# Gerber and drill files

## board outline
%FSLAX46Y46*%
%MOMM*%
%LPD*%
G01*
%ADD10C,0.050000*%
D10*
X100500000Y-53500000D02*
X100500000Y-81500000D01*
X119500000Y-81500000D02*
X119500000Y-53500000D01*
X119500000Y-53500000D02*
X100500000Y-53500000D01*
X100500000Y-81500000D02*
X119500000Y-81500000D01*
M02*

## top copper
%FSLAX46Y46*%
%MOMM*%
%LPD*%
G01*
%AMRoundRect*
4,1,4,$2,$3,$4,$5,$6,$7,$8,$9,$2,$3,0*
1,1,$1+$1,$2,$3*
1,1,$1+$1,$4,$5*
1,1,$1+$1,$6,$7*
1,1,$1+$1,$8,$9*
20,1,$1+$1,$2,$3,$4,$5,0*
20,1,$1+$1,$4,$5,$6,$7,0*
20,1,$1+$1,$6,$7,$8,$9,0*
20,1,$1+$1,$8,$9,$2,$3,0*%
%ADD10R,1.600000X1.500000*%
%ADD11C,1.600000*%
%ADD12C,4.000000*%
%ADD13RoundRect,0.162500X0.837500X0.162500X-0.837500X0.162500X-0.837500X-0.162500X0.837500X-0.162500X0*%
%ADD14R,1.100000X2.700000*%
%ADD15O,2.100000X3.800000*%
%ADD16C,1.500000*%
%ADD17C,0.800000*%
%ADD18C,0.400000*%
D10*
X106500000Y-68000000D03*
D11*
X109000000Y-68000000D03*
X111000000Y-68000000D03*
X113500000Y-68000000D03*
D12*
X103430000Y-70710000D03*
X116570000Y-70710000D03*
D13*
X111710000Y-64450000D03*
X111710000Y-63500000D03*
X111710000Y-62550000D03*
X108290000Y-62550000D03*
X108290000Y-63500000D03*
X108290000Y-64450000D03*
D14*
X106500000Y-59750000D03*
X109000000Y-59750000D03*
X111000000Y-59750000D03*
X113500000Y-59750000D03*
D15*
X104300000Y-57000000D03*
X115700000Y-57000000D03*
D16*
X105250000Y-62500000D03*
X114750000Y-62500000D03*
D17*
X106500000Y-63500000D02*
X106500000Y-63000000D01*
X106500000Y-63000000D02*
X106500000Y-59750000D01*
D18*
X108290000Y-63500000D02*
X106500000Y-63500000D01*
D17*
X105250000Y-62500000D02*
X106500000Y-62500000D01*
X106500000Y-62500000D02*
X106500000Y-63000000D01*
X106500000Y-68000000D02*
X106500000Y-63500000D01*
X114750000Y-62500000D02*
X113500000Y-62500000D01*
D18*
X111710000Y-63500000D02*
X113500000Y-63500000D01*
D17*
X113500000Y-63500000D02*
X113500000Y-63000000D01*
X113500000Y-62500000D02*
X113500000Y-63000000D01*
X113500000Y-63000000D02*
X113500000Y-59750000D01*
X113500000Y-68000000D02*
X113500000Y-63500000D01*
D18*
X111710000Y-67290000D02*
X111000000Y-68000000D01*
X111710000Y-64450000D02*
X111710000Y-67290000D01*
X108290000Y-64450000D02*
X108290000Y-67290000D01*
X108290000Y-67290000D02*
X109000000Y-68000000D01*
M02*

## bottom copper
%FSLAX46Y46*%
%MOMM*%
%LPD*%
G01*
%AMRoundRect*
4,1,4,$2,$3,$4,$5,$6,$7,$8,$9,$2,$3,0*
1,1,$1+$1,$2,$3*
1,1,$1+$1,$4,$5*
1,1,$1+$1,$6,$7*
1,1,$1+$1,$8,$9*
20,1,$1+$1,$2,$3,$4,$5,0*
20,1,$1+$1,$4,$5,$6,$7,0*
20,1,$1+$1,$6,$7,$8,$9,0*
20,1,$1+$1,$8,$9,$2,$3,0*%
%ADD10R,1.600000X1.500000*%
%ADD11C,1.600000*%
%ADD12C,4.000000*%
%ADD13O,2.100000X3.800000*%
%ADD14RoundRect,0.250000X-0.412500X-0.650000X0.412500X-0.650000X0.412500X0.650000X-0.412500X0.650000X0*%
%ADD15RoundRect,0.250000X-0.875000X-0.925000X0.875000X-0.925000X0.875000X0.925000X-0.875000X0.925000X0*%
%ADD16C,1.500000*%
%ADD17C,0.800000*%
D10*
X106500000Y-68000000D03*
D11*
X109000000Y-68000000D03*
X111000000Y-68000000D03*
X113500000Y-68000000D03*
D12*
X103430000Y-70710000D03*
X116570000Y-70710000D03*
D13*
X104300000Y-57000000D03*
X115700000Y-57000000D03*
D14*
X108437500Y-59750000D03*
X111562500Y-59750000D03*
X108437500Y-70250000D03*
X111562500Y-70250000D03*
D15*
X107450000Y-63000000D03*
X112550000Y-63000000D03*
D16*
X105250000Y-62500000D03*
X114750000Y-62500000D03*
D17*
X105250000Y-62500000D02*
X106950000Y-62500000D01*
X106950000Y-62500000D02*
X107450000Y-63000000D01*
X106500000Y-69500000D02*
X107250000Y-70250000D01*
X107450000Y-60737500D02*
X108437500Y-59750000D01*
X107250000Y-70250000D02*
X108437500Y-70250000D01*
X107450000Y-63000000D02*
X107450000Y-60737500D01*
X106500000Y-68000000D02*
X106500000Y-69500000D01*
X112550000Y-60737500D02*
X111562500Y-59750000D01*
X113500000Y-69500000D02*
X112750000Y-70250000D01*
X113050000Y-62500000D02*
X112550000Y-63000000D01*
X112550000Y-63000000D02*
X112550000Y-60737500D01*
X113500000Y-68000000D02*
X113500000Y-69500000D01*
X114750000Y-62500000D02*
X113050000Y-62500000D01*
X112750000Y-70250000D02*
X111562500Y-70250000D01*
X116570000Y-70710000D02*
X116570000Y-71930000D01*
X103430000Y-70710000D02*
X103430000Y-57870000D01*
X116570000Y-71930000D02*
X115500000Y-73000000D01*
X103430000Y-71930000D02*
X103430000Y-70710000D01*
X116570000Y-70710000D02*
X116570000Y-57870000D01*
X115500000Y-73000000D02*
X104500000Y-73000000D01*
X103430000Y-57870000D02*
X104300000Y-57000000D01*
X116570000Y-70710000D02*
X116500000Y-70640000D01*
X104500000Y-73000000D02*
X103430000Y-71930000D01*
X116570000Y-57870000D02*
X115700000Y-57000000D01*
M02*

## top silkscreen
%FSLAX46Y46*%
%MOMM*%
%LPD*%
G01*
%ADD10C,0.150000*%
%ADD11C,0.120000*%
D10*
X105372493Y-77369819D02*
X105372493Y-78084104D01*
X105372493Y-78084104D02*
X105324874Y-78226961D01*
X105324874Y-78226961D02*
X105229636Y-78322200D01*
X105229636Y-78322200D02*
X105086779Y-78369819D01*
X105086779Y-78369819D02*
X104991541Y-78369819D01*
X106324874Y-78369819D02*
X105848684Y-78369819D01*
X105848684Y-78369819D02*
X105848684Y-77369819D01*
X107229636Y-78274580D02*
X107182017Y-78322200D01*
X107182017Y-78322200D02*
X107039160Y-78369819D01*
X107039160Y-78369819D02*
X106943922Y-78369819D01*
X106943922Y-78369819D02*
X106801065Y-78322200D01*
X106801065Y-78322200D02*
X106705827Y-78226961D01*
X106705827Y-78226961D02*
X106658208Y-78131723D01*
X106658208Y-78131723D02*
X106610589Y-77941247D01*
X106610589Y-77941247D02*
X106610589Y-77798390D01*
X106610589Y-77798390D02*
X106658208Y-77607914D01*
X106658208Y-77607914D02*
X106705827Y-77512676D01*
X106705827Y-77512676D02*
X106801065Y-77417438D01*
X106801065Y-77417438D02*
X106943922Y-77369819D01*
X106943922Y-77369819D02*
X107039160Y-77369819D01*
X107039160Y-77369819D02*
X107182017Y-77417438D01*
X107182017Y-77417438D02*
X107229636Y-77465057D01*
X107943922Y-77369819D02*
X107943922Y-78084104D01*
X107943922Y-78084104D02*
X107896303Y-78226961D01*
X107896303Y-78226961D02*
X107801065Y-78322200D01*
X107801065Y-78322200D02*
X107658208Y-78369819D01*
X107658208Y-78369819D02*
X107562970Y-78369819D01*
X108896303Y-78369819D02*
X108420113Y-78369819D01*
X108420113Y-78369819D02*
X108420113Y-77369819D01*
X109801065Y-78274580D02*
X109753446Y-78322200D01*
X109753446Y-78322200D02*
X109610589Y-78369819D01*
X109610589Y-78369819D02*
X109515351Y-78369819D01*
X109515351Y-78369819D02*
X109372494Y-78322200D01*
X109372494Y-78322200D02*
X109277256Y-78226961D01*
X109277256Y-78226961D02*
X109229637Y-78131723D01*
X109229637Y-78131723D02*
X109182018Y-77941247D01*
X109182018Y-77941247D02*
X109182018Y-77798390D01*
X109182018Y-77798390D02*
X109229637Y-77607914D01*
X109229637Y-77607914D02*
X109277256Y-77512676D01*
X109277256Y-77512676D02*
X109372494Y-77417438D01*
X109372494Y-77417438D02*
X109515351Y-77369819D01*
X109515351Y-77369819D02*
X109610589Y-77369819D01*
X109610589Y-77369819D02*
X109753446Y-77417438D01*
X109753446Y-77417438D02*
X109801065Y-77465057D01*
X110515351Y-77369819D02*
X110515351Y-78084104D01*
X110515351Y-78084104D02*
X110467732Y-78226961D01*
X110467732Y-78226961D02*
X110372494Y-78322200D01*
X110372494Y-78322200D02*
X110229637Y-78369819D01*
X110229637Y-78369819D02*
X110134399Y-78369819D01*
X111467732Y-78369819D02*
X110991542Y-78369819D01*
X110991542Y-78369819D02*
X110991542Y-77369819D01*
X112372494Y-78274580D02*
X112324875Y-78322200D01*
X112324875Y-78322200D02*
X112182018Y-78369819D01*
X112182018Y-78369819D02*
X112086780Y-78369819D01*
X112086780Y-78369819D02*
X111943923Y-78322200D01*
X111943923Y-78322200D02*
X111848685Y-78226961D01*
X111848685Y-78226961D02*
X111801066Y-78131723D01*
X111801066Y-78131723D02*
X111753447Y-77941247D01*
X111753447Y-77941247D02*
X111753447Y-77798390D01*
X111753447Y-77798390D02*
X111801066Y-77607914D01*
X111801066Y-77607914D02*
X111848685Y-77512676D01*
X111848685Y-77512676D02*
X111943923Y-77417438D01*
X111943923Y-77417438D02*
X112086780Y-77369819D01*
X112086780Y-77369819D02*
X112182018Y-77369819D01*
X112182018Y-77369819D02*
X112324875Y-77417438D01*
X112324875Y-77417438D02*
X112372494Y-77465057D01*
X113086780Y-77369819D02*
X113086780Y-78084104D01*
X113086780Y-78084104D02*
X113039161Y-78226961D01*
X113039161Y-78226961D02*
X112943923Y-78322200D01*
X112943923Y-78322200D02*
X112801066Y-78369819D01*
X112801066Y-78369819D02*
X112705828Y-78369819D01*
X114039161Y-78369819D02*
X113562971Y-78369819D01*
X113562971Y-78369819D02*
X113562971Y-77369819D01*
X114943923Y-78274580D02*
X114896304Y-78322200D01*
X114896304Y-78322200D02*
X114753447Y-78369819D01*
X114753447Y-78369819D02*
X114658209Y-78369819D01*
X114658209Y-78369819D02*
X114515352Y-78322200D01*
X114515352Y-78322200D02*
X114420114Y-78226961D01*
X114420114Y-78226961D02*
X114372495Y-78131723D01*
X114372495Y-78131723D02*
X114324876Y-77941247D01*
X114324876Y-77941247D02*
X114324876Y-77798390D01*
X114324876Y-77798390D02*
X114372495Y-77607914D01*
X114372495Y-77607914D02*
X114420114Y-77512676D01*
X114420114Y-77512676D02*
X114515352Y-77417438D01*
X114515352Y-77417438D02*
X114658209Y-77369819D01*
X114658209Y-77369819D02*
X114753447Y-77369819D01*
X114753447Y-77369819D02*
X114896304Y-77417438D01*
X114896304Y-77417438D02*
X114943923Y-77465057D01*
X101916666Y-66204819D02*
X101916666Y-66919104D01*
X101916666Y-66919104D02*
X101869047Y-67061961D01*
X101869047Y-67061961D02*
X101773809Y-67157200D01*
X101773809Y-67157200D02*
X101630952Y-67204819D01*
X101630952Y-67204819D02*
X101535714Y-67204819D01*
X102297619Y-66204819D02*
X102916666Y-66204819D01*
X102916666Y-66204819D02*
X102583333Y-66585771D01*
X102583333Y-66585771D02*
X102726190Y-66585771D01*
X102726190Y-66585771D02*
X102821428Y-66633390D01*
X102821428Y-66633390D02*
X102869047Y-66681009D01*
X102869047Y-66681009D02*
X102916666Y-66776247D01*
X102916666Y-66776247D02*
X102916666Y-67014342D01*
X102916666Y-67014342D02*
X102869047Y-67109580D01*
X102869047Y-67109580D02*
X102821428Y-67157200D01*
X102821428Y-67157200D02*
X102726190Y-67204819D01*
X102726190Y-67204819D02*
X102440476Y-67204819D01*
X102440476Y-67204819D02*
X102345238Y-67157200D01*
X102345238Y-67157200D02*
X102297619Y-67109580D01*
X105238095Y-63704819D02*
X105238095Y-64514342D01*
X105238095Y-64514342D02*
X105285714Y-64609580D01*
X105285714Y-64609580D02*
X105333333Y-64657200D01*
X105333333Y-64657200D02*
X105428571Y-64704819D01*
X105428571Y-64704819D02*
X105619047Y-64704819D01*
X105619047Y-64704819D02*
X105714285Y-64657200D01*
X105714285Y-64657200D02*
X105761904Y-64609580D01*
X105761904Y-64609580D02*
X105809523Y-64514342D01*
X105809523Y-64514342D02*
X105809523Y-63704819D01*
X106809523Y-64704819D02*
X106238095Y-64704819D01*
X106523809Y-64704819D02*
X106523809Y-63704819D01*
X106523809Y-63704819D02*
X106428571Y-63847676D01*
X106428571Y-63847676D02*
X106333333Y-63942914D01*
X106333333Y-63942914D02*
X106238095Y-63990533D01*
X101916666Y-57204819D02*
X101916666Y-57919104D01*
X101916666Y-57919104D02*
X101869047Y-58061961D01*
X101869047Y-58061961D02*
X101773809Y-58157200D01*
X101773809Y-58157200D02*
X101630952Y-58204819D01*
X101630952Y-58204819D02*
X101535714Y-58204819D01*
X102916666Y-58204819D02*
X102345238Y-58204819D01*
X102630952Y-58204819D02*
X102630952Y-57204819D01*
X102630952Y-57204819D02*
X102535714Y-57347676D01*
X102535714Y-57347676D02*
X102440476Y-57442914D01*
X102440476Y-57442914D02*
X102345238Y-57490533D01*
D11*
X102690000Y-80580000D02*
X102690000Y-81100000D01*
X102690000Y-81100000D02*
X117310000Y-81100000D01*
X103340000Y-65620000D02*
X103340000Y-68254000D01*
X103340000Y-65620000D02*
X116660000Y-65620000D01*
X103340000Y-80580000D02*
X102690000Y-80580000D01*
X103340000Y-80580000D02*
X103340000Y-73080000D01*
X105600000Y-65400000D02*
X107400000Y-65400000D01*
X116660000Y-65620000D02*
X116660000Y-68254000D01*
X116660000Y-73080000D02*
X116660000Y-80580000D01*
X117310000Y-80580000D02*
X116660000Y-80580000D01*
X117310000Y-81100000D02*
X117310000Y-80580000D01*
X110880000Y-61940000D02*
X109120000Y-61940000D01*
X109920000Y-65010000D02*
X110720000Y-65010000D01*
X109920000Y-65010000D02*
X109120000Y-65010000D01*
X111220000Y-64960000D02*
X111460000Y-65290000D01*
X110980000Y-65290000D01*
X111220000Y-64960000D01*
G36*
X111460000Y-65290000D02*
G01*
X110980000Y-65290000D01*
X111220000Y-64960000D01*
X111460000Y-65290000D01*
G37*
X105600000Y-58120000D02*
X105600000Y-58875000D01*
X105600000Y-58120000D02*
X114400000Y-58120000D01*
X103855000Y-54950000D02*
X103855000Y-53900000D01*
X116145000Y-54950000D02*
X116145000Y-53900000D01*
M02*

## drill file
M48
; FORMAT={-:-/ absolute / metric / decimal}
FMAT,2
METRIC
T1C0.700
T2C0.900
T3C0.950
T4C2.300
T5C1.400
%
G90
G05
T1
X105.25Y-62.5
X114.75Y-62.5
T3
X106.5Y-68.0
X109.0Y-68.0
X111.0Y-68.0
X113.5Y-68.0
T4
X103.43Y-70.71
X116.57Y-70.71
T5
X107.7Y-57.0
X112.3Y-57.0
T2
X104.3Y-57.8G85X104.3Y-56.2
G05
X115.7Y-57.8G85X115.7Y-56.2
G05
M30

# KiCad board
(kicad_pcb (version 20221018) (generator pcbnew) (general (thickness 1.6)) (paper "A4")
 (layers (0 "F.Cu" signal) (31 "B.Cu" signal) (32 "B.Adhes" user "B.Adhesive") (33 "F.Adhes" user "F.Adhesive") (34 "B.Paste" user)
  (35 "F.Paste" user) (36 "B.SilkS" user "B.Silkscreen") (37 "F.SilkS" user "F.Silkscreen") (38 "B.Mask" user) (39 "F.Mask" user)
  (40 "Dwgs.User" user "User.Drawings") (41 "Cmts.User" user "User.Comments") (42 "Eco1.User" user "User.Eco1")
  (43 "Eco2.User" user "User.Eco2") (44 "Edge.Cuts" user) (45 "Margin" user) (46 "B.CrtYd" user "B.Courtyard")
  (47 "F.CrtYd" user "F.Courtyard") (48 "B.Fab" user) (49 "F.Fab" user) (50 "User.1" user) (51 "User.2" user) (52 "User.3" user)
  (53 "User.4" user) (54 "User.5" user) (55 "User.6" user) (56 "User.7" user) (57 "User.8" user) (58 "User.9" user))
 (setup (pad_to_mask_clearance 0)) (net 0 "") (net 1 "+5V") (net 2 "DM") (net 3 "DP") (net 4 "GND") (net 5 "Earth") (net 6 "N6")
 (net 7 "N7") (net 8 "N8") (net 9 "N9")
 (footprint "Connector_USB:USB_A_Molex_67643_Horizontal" (layer "F.Cu") (at 106.5 68)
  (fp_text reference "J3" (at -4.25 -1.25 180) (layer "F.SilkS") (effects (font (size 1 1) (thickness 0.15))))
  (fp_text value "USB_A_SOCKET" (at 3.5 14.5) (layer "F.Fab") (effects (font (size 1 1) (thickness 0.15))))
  (fp_line (start -3.81 12.58) (end -3.81 13.1) (stroke (width 0.12) (type solid)) (layer "F.SilkS"))
  (fp_line (start -3.81 13.1) (end 10.81 13.1) (stroke (width 0.12) (type solid)) (layer "F.SilkS"))
  (fp_line (start -3.16 -2.38) (end -3.16 0.254) (stroke (width 0.12) (type solid)) (layer "F.SilkS"))
  (fp_line (start -3.16 -2.38) (end 10.16 -2.38) (stroke (width 0.12) (type solid)) (layer "F.SilkS"))
  (fp_line (start -3.16 12.58) (end -3.81 12.58) (stroke (width 0.12) (type solid)) (layer "F.SilkS"))
  (fp_line (start -3.16 12.58) (end -3.16 5.08) (stroke (width 0.12) (type solid)) (layer "F.SilkS"))
  (fp_line (start -0.9 -2.6) (end 0.9 -2.6) (stroke (width 0.12) (type solid)) (layer "F.SilkS"))
  (fp_line (start 10.16 -2.38) (end 10.16 0.254) (stroke (width 0.12) (type solid)) (layer "F.SilkS"))
  (fp_line (start 10.16 5.08) (end 10.16 12.58) (stroke (width 0.12) (type solid)) (layer "F.SilkS"))
  (fp_line (start 10.81 12.58) (end 10.16 12.58) (stroke (width 0.12) (type solid)) (layer "F.SilkS"))
  (fp_line (start 10.81 13.1) (end 10.81 12.58) (stroke (width 0.12) (type solid)) (layer "F.SilkS"))
  (pad "1" thru_hole rect (at 0 0) (size 1.6 1.5) (drill 0.95) (layers "*.Cu" "*.Mask") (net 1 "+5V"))
  (pad "2" thru_hole circle (at 2.5 0) (size 1.6 1.6) (drill 0.95) (layers "*.Cu" "*.Mask") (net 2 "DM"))
  (pad "3" thru_hole circle (at 4.5 0) (size 1.6 1.6) (drill 0.95) (layers "*.Cu" "*.Mask") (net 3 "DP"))
  (pad "4" thru_hole circle (at 7 0) (size 1.6 1.6) (drill 0.95) (layers "*.Cu" "*.Mask") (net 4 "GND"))
  (pad "5" thru_hole circle (at -3.07 2.71) (size 4 4) (drill 2.3) (layers "*.Cu" "*.Mask") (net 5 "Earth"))
  (pad "5" thru_hole circle (at 10.07 2.71) (size 4 4) (drill 2.3) (layers "*.Cu" "*.Mask") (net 5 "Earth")))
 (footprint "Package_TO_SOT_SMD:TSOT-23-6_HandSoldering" (layer "F.Cu") (at 110 63.5 180)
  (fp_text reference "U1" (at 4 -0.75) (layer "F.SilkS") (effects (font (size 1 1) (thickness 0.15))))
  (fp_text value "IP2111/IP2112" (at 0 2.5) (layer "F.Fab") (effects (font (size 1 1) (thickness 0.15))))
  (fp_line (start -0.88 1.56) (end 0.88 1.56) (stroke (width 0.12) (type solid)) (layer "F.SilkS"))
  (fp_line (start 0.08 -1.51) (end -0.72 -1.51) (stroke (width 0.12) (type solid)) (layer "F.SilkS"))
  (fp_line (start 0.08 -1.51) (end 0.88 -1.51) (stroke (width 0.12) (type solid)) (layer "F.SilkS"))
  (fp_poly
   (pts (xy -1.22 -1.46) (xy -1.46 -1.79) (xy -0.98 -1.79) (xy -1.22 -1.46)) (stroke (width 0.12) (type solid)) (fill solid)
   (layer "F.SilkS"))
  (pad "1" smd roundrect (at -1.71 -0.95 180) (size 2 0.65) (layers "F.Cu" "F.Paste" "F.Mask") (roundrect_rratio 0.25) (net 3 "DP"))
  (pad "2" smd roundrect (at -1.71 0 180) (size 2 0.65) (layers "F.Cu" "F.Paste" "F.Mask") (roundrect_rratio 0.25) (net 4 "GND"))
  (pad "3" smd roundrect (at -1.71 0.95 180) (size 2 0.65) (layers "F.Cu" "F.Paste" "F.Mask") (roundrect_rratio 0.25) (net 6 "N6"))
  (pad "4" smd roundrect (at 1.71 0.95 180) (size 2 0.65) (layers "F.Cu" "F.Paste" "F.Mask") (roundrect_rratio 0.25) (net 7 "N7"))
  (pad "5" smd roundrect (at 1.71 0 180) (size 2 0.65) (layers "F.Cu" "F.Paste" "F.Mask") (roundrect_rratio 0.25) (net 1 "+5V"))
  (pad "6" smd roundrect (at 1.71 -0.95 180) (size 2 0.65) (layers "F.Cu" "F.Paste" "F.Mask") (roundrect_rratio 0.25) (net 2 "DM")))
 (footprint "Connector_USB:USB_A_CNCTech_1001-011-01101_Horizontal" (layer "F.Cu") (at 110 50.1 90)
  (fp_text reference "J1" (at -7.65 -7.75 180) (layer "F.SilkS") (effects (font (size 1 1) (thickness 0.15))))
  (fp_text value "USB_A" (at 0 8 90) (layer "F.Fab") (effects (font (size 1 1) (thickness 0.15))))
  (fp_line (start -8.02 -4.4) (end -8.775 -4.4) (stroke (width 0.12) (type solid)) (layer "F.SilkS"))
  (fp_line (start -8.02 -4.4) (end -8.02 4.4) (stroke (width 0.12) (type solid)) (layer "F.SilkS"))
  (fp_line (start -4.85 -6.145) (end -3.8 -6.145) (stroke (width 0.12) (type solid)) (layer "F.SilkS"))
  (fp_line (start -4.85 6.145) (end -3.8 6.145) (stroke (width 0.12) (type solid)) (layer "F.SilkS"))
  (pad "" np_thru_hole circle (at -6.9 -2.3 90) (size 1.1 1.1) (drill 1.4) (layers "F&B.Cu" "*.Mask"))
  (pad "" np_thru_hole circle (at -6.9 2.3 90) (size 1.1 1.1) (drill 1.4) (layers "F&B.Cu" "*.Mask"))
  (pad "1" smd rect (at -9.65 -3.5 90) (size 2.7 1.1) (layers "F.Cu" "F.Paste" "F.Mask") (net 1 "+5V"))
  (pad "2" smd rect (at -9.65 -1 90) (size 2.7 1.1) (layers "F.Cu" "F.Paste" "F.Mask") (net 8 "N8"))
  (pad "3" smd rect (at -9.65 1 90) (size 2.7 1.1) (layers "F.Cu" "F.Paste" "F.Mask") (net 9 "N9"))
  (pad "4" smd rect (at -9.65 3.5 90) (size 2.7 1.1) (layers "F.Cu" "F.Paste" "F.Mask") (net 4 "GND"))
  (pad "5" thru_hole oval (at -6.9 -5.7 90) (size 3.8 2.1) (drill oval 2.5 0.9) (layers "*.Cu" "*.Mask") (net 5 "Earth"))
  (pad "5" thru_hole oval (at -6.9 5.7 90) (size 3.8 2.1) (drill oval 2.5 0.9) (layers "*.Cu" "*.Mask") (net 5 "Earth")))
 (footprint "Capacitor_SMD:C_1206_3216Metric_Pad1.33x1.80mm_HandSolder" (layer "B.Cu") (at 110 59.75)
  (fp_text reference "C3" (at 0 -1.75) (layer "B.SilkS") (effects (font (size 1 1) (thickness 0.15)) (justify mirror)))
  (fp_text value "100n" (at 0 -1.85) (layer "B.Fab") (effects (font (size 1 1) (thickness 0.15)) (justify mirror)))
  (pad "1" smd roundrect (at -1.5625 0) (size 1.325 1.8) (layers "B.Cu" "B.Paste" "B.Mask") (roundrect_rratio 0.1886792453) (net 1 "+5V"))
  (pad "2" smd roundrect (at 1.5625 0) (size 1.325 1.8) (layers "B.Cu" "B.Paste" "B.Mask") (roundrect_rratio 0.1886792453) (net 4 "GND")))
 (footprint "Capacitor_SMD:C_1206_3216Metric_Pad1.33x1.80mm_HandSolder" (layer "B.Cu") (at 110 70.25)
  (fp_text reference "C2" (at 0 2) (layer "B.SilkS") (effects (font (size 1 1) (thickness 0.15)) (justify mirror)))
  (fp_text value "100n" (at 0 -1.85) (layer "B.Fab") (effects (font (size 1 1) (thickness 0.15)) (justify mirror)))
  (pad "1" smd roundrect (at -1.5625 0) (size 1.325 1.8) (layers "B.Cu" "B.Paste" "B.Mask") (roundrect_rratio 0.1886792453) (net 1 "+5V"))
  (pad "2" smd roundrect (at 1.5625 0) (size 1.325 1.8) (layers "B.Cu" "B.Paste" "B.Mask") (roundrect_rratio 0.1886792453) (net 4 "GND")))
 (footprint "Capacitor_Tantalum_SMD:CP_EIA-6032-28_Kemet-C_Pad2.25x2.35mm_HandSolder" (layer "B.Cu") (at 110 63)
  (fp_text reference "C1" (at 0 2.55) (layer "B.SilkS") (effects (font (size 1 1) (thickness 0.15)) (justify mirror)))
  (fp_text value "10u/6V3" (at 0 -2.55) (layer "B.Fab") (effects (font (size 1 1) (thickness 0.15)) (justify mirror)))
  (pad "1" smd roundrect (at -2.55 0) (size 2.25 2.35) (layers "B.Cu" "B.Paste" "B.Mask") (roundrect_rratio 0.1111111111) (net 1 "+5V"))
  (pad "2" smd roundrect (at 2.55 0) (size 2.25 2.35) (layers "B.Cu" "B.Paste" "B.Mask") (roundrect_rratio 0.1111111111) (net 4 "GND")))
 (gr_line (start 100.5 53.5) (end 100.5 81.5) (stroke (width 0.05) (type default)) (layer "Edge.Cuts"))
 (gr_line (start 119.5 81.5) (end 119.5 53.5) (stroke (width 0.05) (type default)) (layer "Edge.Cuts"))
 (gr_line (start 119.5 53.5) (end 100.5 53.5) (stroke (width 0.05) (type default)) (layer "Edge.Cuts"))
 (gr_line (start 100.5 81.5) (end 119.5 81.5) (stroke (width 0.05) (type default)) (layer "Edge.Cuts"))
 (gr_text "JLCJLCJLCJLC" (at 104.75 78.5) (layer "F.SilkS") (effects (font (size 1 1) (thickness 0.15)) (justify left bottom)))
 (segment (start 106.5 63.5) (end 106.5 63) (width 0.8) (layer "F.Cu") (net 1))
 (segment (start 106.5 63) (end 106.5 59.75) (width 0.8) (layer "F.Cu") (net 1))
 (segment (start 108.29 63.5) (end 106.5 63.5) (width 0.4) (layer "F.Cu") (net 1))
 (segment (start 105.25 62.5) (end 106.5 62.5) (width 0.8) (layer "F.Cu") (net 1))
 (segment (start 106.5 62.5) (end 106.5 63) (width 0.8) (layer "F.Cu") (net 1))
 (segment (start 106.5 68) (end 106.5 63.5) (width 0.8) (layer "F.Cu") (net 1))
 (via (at 105.25 62.5) (size 1.5) (drill 0.7) (layers "F.Cu" "B.Cu") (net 1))
 (segment (start 105.25 62.5) (end 106.95 62.5) (width 0.8) (layer "B.Cu") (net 1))
 (segment (start 106.95 62.5) (end 107.45 63) (width 0.8) (layer "B.Cu") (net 1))
 (segment (start 106.5 69.5) (end 107.25 70.25) (width 0.8) (layer "B.Cu") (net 1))
 (segment (start 107.45 60.7375) (end 108.4375 59.75) (width 0.8) (layer "B.Cu") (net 1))
 (segment (start 107.25 70.25) (end 108.4375 70.25) (width 0.8) (layer "B.Cu") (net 1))
 (segment (start 107.45 63) (end 107.45 60.7375) (width 0.8) (layer "B.Cu") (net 1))
 (segment (start 106.5 68) (end 106.5 69.5) (width 0.8) (layer "B.Cu") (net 1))
 (segment (start 114.75 62.5) (end 113.5 62.5) (width 0.8) (layer "F.Cu") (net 4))
 (segment (start 111.71 63.5) (end 113.5 63.5) (width 0.4) (layer "F.Cu") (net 4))
 (segment (start 113.5 63.5) (end 113.5 63) (width 0.8) (layer "F.Cu") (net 4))
 (segment (start 113.5 62.5) (end 113.5 63) (width 0.8) (layer "F.Cu") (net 4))
 (segment (start 113.5 63) (end 113.5 59.75) (width 0.8) (layer "F.Cu") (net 4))
 (segment (start 113.5 68) (end 113.5 63.5) (width 0.8) (layer "F.Cu") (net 4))
 (via (at 114.75 62.5) (size 1.5) (drill 0.7) (layers "F.Cu" "B.Cu") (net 4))
 (segment (start 112.55 60.7375) (end 111.5625 59.75) (width 0.8) (layer "B.Cu") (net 4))
 (segment (start 113.5 69.5) (end 112.75 70.25) (width 0.8) (layer "B.Cu") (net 4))
 (segment (start 113.05 62.5) (end 112.55 63) (width 0.8) (layer "B.Cu") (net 4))
 (segment (start 112.55 63) (end 112.55 60.7375) (width 0.8) (layer "B.Cu") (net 4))
 (segment (start 113.5 68) (end 113.5 69.5) (width 0.8) (layer "B.Cu") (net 4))
 (segment (start 114.75 62.5) (end 113.05 62.5) (width 0.8) (layer "B.Cu") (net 4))
 (segment (start 112.75 70.25) (end 111.5625 70.25) (width 0.8) (layer "B.Cu") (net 4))
 (segment (start 116.57 70.71) (end 116.57 71.93) (width 0.8) (layer "B.Cu") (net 5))
 (segment (start 103.43 70.71) (end 103.43 57.87) (width 0.8) (layer "B.Cu") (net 5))
 (segment (start 116.57 71.93) (end 115.5 73) (width 0.8) (layer "B.Cu") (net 5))
 (segment (start 103.43 71.93) (end 103.43 70.71) (width 0.8) (layer "B.Cu") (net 5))
 (segment (start 116.57 70.71) (end 116.57 57.87) (width 0.8) (layer "B.Cu") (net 5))
 (segment (start 115.5 73) (end 104.5 73) (width 0.8) (layer "B.Cu") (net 5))
 (segment (start 103.43 57.87) (end 104.3 57) (width 0.8) (layer "B.Cu") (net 5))
 (segment (start 116.57 70.71) (end 116.5 70.64) (width 0.8) (layer "B.Cu") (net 5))
 (segment (start 104.5 73) (end 103.43 71.93) (width 0.8) (layer "B.Cu") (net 5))
 (segment (start 116.57 57.87) (end 115.7 57) (width 0.8) (layer "B.Cu") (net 5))
 (segment (start 111.71 67.29) (end 111 68) (width 0.4) (layer "F.Cu") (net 3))
 (segment (start 111.71 64.45) (end 111.71 67.29) (width 0.4) (layer "F.Cu") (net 3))
 (segment (start 108.29 64.45) (end 108.29 67.29) (width 0.4) (layer "F.Cu") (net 2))
 (segment (start 108.29 67.29) (end 109 68) (width 0.4) (layer "F.Cu") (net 2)))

